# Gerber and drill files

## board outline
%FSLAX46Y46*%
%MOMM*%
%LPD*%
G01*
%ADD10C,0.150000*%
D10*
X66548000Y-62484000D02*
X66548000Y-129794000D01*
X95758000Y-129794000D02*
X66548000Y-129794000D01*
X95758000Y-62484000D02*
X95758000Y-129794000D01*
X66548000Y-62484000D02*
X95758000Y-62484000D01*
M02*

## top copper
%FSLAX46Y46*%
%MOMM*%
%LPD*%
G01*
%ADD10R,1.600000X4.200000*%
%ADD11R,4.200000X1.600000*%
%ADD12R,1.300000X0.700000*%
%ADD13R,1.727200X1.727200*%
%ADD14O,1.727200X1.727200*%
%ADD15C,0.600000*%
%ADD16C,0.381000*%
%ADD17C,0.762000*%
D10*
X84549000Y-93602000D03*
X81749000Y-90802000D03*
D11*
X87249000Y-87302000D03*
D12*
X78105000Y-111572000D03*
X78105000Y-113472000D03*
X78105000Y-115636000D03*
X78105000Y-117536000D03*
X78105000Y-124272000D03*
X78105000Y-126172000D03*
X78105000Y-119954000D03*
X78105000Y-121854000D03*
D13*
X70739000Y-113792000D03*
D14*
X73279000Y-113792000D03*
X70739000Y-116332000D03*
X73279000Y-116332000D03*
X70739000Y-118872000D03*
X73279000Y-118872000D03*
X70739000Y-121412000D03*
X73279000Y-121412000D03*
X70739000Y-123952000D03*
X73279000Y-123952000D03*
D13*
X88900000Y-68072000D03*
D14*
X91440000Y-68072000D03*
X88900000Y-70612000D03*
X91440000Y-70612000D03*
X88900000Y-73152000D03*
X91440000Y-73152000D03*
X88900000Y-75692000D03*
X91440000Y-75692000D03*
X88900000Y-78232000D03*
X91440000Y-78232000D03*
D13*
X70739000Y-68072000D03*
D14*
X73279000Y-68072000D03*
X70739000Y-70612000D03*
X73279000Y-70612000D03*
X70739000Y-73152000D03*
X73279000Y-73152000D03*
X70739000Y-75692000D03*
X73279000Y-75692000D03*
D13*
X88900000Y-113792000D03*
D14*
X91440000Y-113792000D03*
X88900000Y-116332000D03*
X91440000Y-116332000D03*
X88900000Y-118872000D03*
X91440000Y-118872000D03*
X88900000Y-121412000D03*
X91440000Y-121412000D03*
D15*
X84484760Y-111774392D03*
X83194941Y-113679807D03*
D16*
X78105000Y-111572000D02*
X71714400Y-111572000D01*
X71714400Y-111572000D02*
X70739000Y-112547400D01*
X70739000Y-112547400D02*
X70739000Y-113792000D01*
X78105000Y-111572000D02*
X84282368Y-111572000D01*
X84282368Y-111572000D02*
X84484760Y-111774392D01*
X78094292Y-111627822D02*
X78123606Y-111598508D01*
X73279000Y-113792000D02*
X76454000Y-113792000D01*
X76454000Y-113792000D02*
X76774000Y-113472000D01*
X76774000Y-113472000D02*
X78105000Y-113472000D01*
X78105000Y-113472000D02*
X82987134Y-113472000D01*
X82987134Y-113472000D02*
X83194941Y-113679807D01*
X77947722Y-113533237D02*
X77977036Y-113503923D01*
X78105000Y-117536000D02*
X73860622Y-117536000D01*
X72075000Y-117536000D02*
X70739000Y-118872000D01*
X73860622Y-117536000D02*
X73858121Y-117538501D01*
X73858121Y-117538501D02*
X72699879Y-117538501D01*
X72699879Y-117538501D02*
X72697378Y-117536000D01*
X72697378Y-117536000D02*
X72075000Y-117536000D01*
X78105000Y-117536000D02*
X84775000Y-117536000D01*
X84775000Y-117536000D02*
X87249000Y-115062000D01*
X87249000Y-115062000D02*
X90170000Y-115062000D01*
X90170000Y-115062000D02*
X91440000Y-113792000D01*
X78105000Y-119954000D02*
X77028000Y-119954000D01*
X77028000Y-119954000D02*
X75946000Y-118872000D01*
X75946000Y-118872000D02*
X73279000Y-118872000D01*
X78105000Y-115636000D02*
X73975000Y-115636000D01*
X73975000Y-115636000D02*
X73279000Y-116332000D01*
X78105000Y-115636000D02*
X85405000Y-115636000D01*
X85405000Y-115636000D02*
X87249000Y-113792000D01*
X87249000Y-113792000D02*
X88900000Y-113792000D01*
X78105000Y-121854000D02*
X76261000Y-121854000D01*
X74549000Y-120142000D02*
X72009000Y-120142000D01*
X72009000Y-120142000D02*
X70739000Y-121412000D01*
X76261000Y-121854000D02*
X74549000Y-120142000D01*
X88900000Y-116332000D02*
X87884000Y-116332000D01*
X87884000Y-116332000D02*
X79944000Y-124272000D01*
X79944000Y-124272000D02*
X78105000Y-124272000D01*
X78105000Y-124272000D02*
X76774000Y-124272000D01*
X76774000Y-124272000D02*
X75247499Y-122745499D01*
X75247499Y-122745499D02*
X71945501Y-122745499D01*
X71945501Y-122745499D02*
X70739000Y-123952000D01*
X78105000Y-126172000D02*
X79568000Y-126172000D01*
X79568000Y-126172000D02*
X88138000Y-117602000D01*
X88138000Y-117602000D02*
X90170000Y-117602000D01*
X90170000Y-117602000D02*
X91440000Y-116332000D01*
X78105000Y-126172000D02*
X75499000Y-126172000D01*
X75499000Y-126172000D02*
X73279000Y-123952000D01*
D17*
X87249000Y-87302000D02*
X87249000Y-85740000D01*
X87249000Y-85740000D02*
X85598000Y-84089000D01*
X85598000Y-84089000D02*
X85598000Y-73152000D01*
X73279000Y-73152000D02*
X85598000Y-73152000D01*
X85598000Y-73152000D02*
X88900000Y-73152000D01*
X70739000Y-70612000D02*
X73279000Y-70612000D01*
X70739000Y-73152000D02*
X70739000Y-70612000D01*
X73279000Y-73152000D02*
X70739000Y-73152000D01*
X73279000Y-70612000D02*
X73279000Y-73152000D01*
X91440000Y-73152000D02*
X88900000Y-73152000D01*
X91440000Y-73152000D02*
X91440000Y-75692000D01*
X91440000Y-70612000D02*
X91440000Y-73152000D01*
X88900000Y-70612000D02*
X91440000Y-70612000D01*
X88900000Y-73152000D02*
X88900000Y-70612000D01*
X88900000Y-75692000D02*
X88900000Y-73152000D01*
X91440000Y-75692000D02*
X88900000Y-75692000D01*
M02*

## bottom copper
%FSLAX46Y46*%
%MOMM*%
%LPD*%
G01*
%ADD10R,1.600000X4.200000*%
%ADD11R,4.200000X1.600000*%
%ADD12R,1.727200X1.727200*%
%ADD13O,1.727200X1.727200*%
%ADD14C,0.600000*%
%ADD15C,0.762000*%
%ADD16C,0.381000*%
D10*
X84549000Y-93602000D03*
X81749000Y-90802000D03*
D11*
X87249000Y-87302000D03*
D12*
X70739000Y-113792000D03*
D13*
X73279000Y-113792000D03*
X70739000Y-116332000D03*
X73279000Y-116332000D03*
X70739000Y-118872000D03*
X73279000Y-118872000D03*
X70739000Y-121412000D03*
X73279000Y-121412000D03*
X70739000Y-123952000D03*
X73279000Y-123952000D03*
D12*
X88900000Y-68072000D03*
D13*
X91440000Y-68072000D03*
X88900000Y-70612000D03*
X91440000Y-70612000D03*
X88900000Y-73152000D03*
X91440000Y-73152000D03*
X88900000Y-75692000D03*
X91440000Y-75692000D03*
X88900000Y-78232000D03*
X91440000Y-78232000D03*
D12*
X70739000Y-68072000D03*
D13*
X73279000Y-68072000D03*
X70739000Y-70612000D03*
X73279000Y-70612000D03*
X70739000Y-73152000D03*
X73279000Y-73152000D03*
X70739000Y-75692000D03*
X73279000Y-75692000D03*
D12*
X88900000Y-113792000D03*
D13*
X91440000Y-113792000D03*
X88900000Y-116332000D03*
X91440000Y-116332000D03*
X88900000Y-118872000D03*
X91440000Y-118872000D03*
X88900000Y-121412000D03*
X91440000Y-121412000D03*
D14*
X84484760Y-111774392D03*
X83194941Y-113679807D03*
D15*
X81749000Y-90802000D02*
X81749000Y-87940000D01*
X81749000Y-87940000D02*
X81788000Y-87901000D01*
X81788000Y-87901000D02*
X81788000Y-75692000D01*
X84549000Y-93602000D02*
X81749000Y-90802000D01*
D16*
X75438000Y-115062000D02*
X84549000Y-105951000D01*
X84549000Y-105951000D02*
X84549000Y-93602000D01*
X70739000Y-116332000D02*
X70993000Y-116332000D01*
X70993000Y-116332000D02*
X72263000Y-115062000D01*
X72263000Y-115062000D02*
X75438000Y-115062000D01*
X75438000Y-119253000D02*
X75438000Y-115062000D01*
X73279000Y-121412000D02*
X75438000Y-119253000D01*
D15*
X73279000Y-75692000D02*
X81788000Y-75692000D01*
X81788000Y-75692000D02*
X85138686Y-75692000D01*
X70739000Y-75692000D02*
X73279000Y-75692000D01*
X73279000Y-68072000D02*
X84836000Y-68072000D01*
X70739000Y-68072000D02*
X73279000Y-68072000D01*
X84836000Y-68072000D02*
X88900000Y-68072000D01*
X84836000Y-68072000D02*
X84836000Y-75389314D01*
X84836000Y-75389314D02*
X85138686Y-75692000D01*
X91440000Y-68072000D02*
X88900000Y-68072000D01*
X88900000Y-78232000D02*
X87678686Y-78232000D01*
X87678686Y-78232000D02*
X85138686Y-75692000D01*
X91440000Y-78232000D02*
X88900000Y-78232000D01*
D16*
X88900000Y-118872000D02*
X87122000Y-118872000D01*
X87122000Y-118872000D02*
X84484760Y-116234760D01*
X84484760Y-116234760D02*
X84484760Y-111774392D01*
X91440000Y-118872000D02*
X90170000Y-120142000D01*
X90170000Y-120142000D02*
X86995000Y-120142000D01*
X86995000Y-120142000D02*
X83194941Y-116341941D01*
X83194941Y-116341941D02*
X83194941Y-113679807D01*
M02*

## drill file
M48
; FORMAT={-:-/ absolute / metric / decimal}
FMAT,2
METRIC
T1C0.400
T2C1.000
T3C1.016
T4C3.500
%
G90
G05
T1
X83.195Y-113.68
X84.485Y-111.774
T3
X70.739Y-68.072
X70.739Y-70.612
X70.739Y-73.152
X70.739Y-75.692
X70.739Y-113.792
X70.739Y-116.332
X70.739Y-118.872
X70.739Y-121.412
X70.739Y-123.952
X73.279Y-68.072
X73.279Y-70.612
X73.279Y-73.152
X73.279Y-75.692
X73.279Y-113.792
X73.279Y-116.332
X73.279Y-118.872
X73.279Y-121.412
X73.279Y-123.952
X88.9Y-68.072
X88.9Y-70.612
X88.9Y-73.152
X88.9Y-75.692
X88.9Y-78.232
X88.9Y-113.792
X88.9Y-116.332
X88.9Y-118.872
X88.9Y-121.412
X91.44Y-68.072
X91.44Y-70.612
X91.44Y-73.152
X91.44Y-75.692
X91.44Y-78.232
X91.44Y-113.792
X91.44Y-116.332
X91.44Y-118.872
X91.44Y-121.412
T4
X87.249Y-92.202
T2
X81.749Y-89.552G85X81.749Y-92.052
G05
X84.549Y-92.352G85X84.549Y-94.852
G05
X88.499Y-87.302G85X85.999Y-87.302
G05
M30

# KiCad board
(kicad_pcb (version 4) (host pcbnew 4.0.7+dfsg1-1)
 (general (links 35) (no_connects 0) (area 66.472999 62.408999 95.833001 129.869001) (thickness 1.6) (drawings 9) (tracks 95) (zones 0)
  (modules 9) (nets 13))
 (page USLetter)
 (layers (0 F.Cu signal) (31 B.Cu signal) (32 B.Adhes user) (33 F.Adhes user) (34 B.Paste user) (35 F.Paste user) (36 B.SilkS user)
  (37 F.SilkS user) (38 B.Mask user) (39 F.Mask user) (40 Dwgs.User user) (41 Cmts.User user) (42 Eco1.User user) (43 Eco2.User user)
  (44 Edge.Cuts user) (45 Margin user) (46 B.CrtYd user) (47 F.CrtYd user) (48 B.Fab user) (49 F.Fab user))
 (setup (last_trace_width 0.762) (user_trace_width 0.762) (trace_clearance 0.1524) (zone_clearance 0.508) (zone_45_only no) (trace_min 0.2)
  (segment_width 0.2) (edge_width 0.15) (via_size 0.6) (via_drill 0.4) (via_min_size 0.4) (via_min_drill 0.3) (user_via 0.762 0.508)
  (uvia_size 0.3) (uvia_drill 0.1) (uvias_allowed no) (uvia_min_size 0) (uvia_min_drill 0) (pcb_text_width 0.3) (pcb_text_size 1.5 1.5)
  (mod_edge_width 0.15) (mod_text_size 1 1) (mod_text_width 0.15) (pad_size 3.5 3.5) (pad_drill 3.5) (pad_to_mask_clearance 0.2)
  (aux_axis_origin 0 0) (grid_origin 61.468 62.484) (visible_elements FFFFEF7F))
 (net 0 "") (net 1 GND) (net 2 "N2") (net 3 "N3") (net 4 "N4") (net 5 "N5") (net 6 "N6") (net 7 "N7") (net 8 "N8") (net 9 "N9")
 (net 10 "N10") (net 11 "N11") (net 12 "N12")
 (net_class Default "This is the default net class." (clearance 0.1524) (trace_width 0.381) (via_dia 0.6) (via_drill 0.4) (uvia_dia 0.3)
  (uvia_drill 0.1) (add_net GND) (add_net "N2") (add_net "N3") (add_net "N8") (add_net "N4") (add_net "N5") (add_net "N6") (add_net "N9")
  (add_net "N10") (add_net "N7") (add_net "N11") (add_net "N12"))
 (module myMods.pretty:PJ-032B (layer F.Cu) (at 87.249 87.302 270)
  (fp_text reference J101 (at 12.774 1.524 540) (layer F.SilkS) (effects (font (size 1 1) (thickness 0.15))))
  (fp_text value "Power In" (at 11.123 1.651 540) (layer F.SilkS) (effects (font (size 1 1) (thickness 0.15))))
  (pad 3 thru_hole rect (at 6.3 2.7) (size 1.6 4.2) (drill oval 1 3.5) (layers *.Cu *.Mask F.SilkS) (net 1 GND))
  (pad 2 thru_hole rect (at 3.5 5.5) (size 1.6 4.2) (drill oval 1 3.5) (layers *.Cu *.Mask F.SilkS) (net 1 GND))
  (pad 1 thru_hole rect (at 0 0 270) (size 1.6 4.2) (drill oval 1 3.5) (layers *.Cu *.Mask F.SilkS) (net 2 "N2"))
  (pad "" np_thru_hole circle (at 4.9 0) (size 3.5 3.5) (drill 3.5) (layers *.Cu *.Mask F.SilkS)))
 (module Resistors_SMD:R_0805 (layer F.Cu) (at 78.105 112.522 270)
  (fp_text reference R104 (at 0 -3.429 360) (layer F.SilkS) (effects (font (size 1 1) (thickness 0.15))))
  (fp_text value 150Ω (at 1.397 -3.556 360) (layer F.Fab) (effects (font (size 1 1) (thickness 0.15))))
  (pad 1 smd rect (at -0.95 0 270) (size 0.7 1.3) (layers F.Cu F.Paste F.Mask) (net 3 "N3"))
  (pad 2 smd rect (at 0.95 0 270) (size 0.7 1.3) (layers F.Cu F.Paste F.Mask) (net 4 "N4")))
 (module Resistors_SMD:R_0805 (layer F.Cu) (at 78.105 116.586 270)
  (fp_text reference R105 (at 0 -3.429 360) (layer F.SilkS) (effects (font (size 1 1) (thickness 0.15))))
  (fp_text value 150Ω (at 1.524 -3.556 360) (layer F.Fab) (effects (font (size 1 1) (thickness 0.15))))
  (pad 1 smd rect (at -0.95 0 270) (size 0.7 1.3) (layers F.Cu F.Paste F.Mask) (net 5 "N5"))
  (pad 2 smd rect (at 0.95 0 270) (size 0.7 1.3) (layers F.Cu F.Paste F.Mask) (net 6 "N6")))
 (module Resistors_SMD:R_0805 (layer F.Cu) (at 78.105 125.222 270)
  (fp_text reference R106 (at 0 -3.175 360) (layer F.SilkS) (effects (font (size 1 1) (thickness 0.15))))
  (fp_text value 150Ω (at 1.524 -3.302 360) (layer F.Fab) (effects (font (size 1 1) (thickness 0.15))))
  (pad 1 smd rect (at -0.95 0 270) (size 0.7 1.3) (layers F.Cu F.Paste F.Mask) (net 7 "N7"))
  (pad 2 smd rect (at 0.95 0 270) (size 0.7 1.3) (layers F.Cu F.Paste F.Mask) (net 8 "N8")))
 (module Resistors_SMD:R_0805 (layer F.Cu) (at 78.105 120.904 270)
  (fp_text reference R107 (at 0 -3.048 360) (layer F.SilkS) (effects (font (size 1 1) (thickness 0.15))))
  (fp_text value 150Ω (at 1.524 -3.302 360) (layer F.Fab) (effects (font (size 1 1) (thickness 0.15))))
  (pad 1 smd rect (at -0.95 0 270) (size 0.7 1.3) (layers F.Cu F.Paste F.Mask) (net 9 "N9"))
  (pad 2 smd rect (at 0.95 0 270) (size 0.7 1.3) (layers F.Cu F.Paste F.Mask) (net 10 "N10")))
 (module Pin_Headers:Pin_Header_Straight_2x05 (layer F.Cu) (at 70.739 113.792)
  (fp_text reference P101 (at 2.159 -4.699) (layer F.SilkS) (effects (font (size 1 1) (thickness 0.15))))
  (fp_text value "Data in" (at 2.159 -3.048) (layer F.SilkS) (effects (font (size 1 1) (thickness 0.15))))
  (pad 1 thru_hole rect (at 0 0) (size 1.7272 1.7272) (drill 1.016) (layers *.Cu *.Mask F.SilkS) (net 3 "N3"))
  (pad 2 thru_hole oval (at 2.54 0) (size 1.7272 1.7272) (drill 1.016) (layers *.Cu *.Mask F.SilkS) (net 4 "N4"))
  (pad 3 thru_hole oval (at 0 2.54) (size 1.7272 1.7272) (drill 1.016) (layers *.Cu *.Mask F.SilkS) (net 1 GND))
  (pad 4 thru_hole oval (at 2.54 2.54) (size 1.7272 1.7272) (drill 1.016) (layers *.Cu *.Mask F.SilkS) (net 5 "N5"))
  (pad 5 thru_hole oval (at 0 5.08) (size 1.7272 1.7272) (drill 1.016) (layers *.Cu *.Mask F.SilkS) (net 6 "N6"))
  (pad 6 thru_hole oval (at 2.54 5.08) (size 1.7272 1.7272) (drill 1.016) (layers *.Cu *.Mask F.SilkS) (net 9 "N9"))
  (pad 7 thru_hole oval (at 0 7.62) (size 1.7272 1.7272) (drill 1.016) (layers *.Cu *.Mask F.SilkS) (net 10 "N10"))
  (pad 8 thru_hole oval (at 2.54 7.62) (size 1.7272 1.7272) (drill 1.016) (layers *.Cu *.Mask F.SilkS) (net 1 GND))
  (pad 9 thru_hole oval (at 0 10.16) (size 1.7272 1.7272) (drill 1.016) (layers *.Cu *.Mask F.SilkS) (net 7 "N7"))
  (pad 10 thru_hole oval (at 2.54 10.16) (size 1.7272 1.7272) (drill 1.016) (layers *.Cu *.Mask F.SilkS) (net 8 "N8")))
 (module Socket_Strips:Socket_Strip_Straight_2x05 (layer B.Cu) (at 88.9 68.072 270)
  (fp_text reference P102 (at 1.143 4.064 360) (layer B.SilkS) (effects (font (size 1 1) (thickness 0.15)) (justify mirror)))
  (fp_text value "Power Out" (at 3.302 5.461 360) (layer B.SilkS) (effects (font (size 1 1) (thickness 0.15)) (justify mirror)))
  (pad 1 thru_hole rect (at 0 0 270) (size 1.7272 1.7272) (drill 1.016) (layers *.Cu *.Mask B.SilkS) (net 1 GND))
  (pad 2 thru_hole oval (at 0 -2.54 270) (size 1.7272 1.7272) (drill 1.016) (layers *.Cu *.Mask B.SilkS) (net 1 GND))
  (pad 3 thru_hole oval (at 2.54 0 270) (size 1.7272 1.7272) (drill 1.016) (layers *.Cu *.Mask B.SilkS) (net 2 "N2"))
  (pad 4 thru_hole oval (at 2.54 -2.54 270) (size 1.7272 1.7272) (drill 1.016) (layers *.Cu *.Mask B.SilkS) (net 2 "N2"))
  (pad 5 thru_hole oval (at 5.08 0 270) (size 1.7272 1.7272) (drill 1.016) (layers *.Cu *.Mask B.SilkS) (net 2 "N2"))
  (pad 6 thru_hole oval (at 5.08 -2.54 270) (size 1.7272 1.7272) (drill 1.016) (layers *.Cu *.Mask B.SilkS) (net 2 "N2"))
  (pad 7 thru_hole oval (at 7.62 0 270) (size 1.7272 1.7272) (drill 1.016) (layers *.Cu *.Mask B.SilkS) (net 2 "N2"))
  (pad 8 thru_hole oval (at 7.62 -2.54 270) (size 1.7272 1.7272) (drill 1.016) (layers *.Cu *.Mask B.SilkS) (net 2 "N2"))
  (pad 9 thru_hole oval (at 10.16 0 270) (size 1.7272 1.7272) (drill 1.016) (layers *.Cu *.Mask B.SilkS) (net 1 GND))
  (pad 10 thru_hole oval (at 10.16 -2.54 270) (size 1.7272 1.7272) (drill 1.016) (layers *.Cu *.Mask B.SilkS) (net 1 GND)))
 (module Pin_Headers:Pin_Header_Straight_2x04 (layer F.Cu) (at 70.739 68.072)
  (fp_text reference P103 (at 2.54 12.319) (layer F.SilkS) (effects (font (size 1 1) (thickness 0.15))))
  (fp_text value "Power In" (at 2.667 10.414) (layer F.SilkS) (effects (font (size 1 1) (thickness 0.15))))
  (pad 1 thru_hole rect (at 0 0) (size 1.7272 1.7272) (drill 1.016) (layers *.Cu *.Mask F.SilkS) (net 1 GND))
  (pad 2 thru_hole oval (at 2.54 0) (size 1.7272 1.7272) (drill 1.016) (layers *.Cu *.Mask F.SilkS) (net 1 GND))
  (pad 3 thru_hole oval (at 0 2.54) (size 1.7272 1.7272) (drill 1.016) (layers *.Cu *.Mask F.SilkS) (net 2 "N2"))
  (pad 4 thru_hole oval (at 2.54 2.54) (size 1.7272 1.7272) (drill 1.016) (layers *.Cu *.Mask F.SilkS) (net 2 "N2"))
  (pad 5 thru_hole oval (at 0 5.08) (size 1.7272 1.7272) (drill 1.016) (layers *.Cu *.Mask F.SilkS) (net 2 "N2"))
  (pad 6 thru_hole oval (at 2.54 5.08) (size 1.7272 1.7272) (drill 1.016) (layers *.Cu *.Mask F.SilkS) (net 2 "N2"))
  (pad 7 thru_hole oval (at 0 7.62) (size 1.7272 1.7272) (drill 1.016) (layers *.Cu *.Mask F.SilkS) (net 1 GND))
  (pad 8 thru_hole oval (at 2.54 7.62) (size 1.7272 1.7272) (drill 1.016) (layers *.Cu *.Mask F.SilkS) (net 1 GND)))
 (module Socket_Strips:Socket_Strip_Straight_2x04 (layer B.Cu) (at 88.9 113.792 270)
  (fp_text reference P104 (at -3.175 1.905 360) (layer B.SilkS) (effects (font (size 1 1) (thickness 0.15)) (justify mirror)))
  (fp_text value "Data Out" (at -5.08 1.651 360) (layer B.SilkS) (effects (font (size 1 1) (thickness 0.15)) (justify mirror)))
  (pad 1 thru_hole rect (at 0 0 270) (size 1.7272 1.7272) (drill 1.016) (layers *.Cu *.Mask B.SilkS) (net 5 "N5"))
  (pad 2 thru_hole oval (at 0 -2.54 270) (size 1.7272 1.7272) (drill 1.016) (layers *.Cu *.Mask B.SilkS) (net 6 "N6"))
  (pad 3 thru_hole oval (at 2.54 0 270) (size 1.7272 1.7272) (drill 1.016) (layers *.Cu *.Mask B.SilkS) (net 7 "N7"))
  (pad 4 thru_hole oval (at 2.54 -2.54 270) (size 1.7272 1.7272) (drill 1.016) (layers *.Cu *.Mask B.SilkS) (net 8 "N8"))
  (pad 5 thru_hole oval (at 5.08 0 270) (size 1.7272 1.7272) (drill 1.016) (layers *.Cu *.Mask B.SilkS) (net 3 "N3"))
  (pad 6 thru_hole oval (at 5.08 -2.54 270) (size 1.7272 1.7272) (drill 1.016) (layers *.Cu *.Mask B.SilkS) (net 4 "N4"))
  (pad 7 thru_hole oval (at 7.62 0 270) (size 1.7272 1.7272) (drill 1.016) (layers *.Cu *.Mask B.SilkS) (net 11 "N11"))
  (pad 8 thru_hole oval (at 7.62 -2.54 270) (size 1.7272 1.7272) (drill 1.016) (layers *.Cu *.Mask B.SilkS) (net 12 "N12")))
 (gr_line (start 66.548 62.484) (end 66.548 129.794) (angle 90) (layer Edge.Cuts) (width 0.15))
 (gr_line (start 95.758 129.794) (end 66.548 129.794) (angle 90) (layer Edge.Cuts) (width 0.15))
 (gr_line (start 95.758 62.484) (end 95.758 129.794) (angle 90) (layer Edge.Cuts) (width 0.15))
 (gr_line (start 66.548 62.484) (end 95.758 62.484) (angle 90) (layer Edge.Cuts) (width 0.15))
 (segment (start 81.749 90.802) (end 81.749 87.94) (width 0.762) (layer B.Cu) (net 1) (status 10))
 (segment (start 81.749 87.94) (end 81.788 87.901) (width 0.762) (layer B.Cu) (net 1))
 (segment (start 81.788 87.901) (end 81.788 75.692) (width 0.762) (layer B.Cu) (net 1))
 (segment (start 84.549 93.602) (end 81.749 90.802) (width 0.762) (layer B.Cu) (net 1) (status 30))
 (segment (start 75.438 115.062) (end 84.549 105.951) (width 0.381) (layer B.Cu) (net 1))
 (segment (start 84.549 105.951) (end 84.549 93.602) (width 0.381) (layer B.Cu) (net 1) (status 20))
 (segment (start 70.739 116.332) (end 70.993 116.332) (width 0.381) (layer B.Cu) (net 1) (status 30))
 (segment (start 70.993 116.332) (end 72.263 115.062) (width 0.381) (layer B.Cu) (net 1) (status 10))
 (segment (start 72.263 115.062) (end 75.438 115.062) (width 0.381) (layer B.Cu) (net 1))
 (segment (start 75.438 119.253) (end 75.438 115.062) (width 0.381) (layer B.Cu) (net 1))
 (segment (start 73.279 121.412) (end 75.438 119.253) (width 0.381) (layer B.Cu) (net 1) (status 10))
 (segment (start 73.279 75.692) (end 81.788 75.692) (width 0.762) (layer B.Cu) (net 1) (status 10))
 (segment (start 81.788 75.692) (end 85.138686 75.692) (width 0.762) (layer B.Cu) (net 1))
 (segment (start 70.739 75.692) (end 73.279 75.692) (width 0.762) (layer B.Cu) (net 1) (status 30))
 (segment (start 73.279 68.072) (end 84.836 68.072) (width 0.762) (layer B.Cu) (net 1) (status 10))
 (segment (start 70.739 68.072) (end 73.279 68.072) (width 0.762) (layer B.Cu) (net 1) (status 30))
 (segment (start 84.836 68.072) (end 88.9 68.072) (width 0.762) (layer B.Cu) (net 1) (status 20))
 (segment (start 84.836 68.072) (end 84.836 75.389314) (width 0.762) (layer B.Cu) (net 1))
 (segment (start 84.836 75.389314) (end 85.138686 75.692) (width 0.762) (layer B.Cu) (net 1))
 (segment (start 91.44 68.072) (end 88.9 68.072) (width 0.762) (layer B.Cu) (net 1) (status 30))
 (segment (start 88.9 78.232) (end 87.678686 78.232) (width 0.762) (layer B.Cu) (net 1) (status 10))
 (segment (start 87.678686 78.232) (end 85.138686 75.692) (width 0.762) (layer B.Cu) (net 1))
 (segment (start 91.44 78.232) (end 88.9 78.232) (width 0.762) (layer B.Cu) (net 1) (status 30))
 (segment (start 88.9 118.872) (end 87.122 118.872) (width 0.381) (layer B.Cu) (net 3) (status 10))
 (segment (start 87.122 118.872) (end 84.48476 116.23476) (width 0.381) (layer B.Cu) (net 3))
 (segment (start 84.48476 116.23476) (end 84.48476 111.774392) (width 0.381) (layer B.Cu) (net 3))
 (segment (start 78.105 111.572) (end 71.7144 111.572) (width 0.381) (layer F.Cu) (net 3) (status 10))
 (segment (start 71.7144 111.572) (end 70.739 112.5474) (width 0.381) (layer F.Cu) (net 3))
 (segment (start 70.739 112.5474) (end 70.739 113.792) (width 0.381) (layer F.Cu) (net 3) (status 20))
 (segment (start 78.105 111.572) (end 84.282368 111.572) (width 0.381) (layer F.Cu) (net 3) (status 10))
 (segment (start 84.282368 111.572) (end 84.48476 111.774392) (width 0.381) (layer F.Cu) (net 3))
 (segment (start 78.094292 111.627822) (end 78.123606 111.598508) (width 0.381) (layer F.Cu) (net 3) (status 30))
 (via (at 84.48476 111.774392) (size 0.6) (drill 0.4) (layers F.Cu B.Cu) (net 3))
 (segment (start 91.44 118.872) (end 90.17 120.142) (width 0.381) (layer B.Cu) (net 4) (status 10))
 (segment (start 90.17 120.142) (end 86.995 120.142) (width 0.381) (layer B.Cu) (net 4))
 (segment (start 86.995 120.142) (end 83.194941 116.341941) (width 0.381) (layer B.Cu) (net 4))
 (segment (start 83.194941 116.341941) (end 83.194941 113.679807) (width 0.381) (layer B.Cu) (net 4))
 (segment (start 73.279 113.792) (end 76.454 113.792) (width 0.381) (layer F.Cu) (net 4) (status 10))
 (segment (start 76.454 113.792) (end 76.774 113.472) (width 0.381) (layer F.Cu) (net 4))
 (segment (start 76.774 113.472) (end 78.105 113.472) (width 0.381) (layer F.Cu) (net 4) (status 20))
 (segment (start 78.105 113.472) (end 82.987134 113.472) (width 0.381) (layer F.Cu) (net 4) (status 10))
 (segment (start 82.987134 113.472) (end 83.194941 113.679807) (width 0.381) (layer F.Cu) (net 4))
 (segment (start 77.947722 113.533237) (end 77.977036 113.503923) (width 0.381) (layer F.Cu) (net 4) (status 30))
 (via (at 83.194941 113.679807) (size 0.6) (drill 0.4) (layers F.Cu B.Cu) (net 4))
 (segment (start 78.105 117.536) (end 73.860622 117.536) (width 0.381) (layer F.Cu) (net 6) (status 10))
 (segment (start 72.075 117.536) (end 70.739 118.872) (width 0.381) (layer F.Cu) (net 6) (status 20))
 (segment (start 73.860622 117.536) (end 73.858121 117.538501) (width 0.381) (layer F.Cu) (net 6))
 (segment (start 73.858121 117.538501) (end 72.699879 117.538501) (width 0.381) (layer F.Cu) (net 6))
 (segment (start 72.699879 117.538501) (end 72.697378 117.536) (width 0.381) (layer F.Cu) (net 6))
 (segment (start 72.697378 117.536) (end 72.075 117.536) (width 0.381) (layer F.Cu) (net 6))
 (segment (start 78.105 117.536) (end 84.775 117.536) (width 0.381) (layer F.Cu) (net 6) (status 10))
 (segment (start 84.775 117.536) (end 87.249 115.062) (width 0.381) (layer F.Cu) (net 6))
 (segment (start 87.249 115.062) (end 90.17 115.062) (width 0.381) (layer F.Cu) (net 6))
 (segment (start 90.17 115.062) (end 91.44 113.792) (width 0.381) (layer F.Cu) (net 6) (status 20))
 (segment (start 78.105 119.954) (end 77.028 119.954) (width 0.381) (layer F.Cu) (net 9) (status 10))
 (segment (start 77.028 119.954) (end 75.946 118.872) (width 0.381) (layer F.Cu) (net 9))
 (segment (start 75.946 118.872) (end 73.279 118.872) (width 0.381) (layer F.Cu) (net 9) (status 20))
 (segment (start 78.105 115.636) (end 73.975 115.636) (width 0.381) (layer F.Cu) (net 5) (status 10))
 (segment (start 73.975 115.636) (end 73.279 116.332) (width 0.381) (layer F.Cu) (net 5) (status 20))
 (segment (start 78.105 115.636) (end 85.405 115.636) (width 0.381) (layer F.Cu) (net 5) (status 10))
 (segment (start 85.405 115.636) (end 87.249 113.792) (width 0.381) (layer F.Cu) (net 5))
 (segment (start 87.249 113.792) (end 88.9 113.792) (width 0.381) (layer F.Cu) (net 5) (status 20))
 (segment (start 78.105 121.854) (end 76.261 121.854) (width 0.381) (layer F.Cu) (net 10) (status 10))
 (segment (start 74.549 120.142) (end 72.009 120.142) (width 0.381) (layer F.Cu) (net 10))
 (segment (start 72.009 120.142) (end 70.739 121.412) (width 0.381) (layer F.Cu) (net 10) (status 20))
 (segment (start 76.261 121.854) (end 74.549 120.142) (width 0.381) (layer F.Cu) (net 10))
 (segment (start 88.9 116.332) (end 87.884 116.332) (width 0.381) (layer F.Cu) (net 7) (status 10))
 (segment (start 87.884 116.332) (end 79.944 124.272) (width 0.381) (layer F.Cu) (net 7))
 (segment (start 79.944 124.272) (end 78.105 124.272) (width 0.381) (layer F.Cu) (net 7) (status 20))
 (segment (start 78.105 124.272) (end 76.774 124.272) (width 0.381) (layer F.Cu) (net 7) (status 10))
 (segment (start 76.774 124.272) (end 75.247499 122.745499) (width 0.381) (layer F.Cu) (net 7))
 (segment (start 75.247499 122.745499) (end 71.945501 122.745499) (width 0.381) (layer F.Cu) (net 7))
 (segment (start 71.945501 122.745499) (end 70.739 123.952) (width 0.381) (layer F.Cu) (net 7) (status 20))
 (segment (start 78.105 126.172) (end 79.568 126.172) (width 0.381) (layer F.Cu) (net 8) (status 10))
 (segment (start 79.568 126.172) (end 88.138 117.602) (width 0.381) (layer F.Cu) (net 8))
 (segment (start 88.138 117.602) (end 90.17 117.602) (width 0.381) (layer F.Cu) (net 8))
 (segment (start 90.17 117.602) (end 91.44 116.332) (width 0.381) (layer F.Cu) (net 8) (status 20))
 (segment (start 78.105 126.172) (end 75.499 126.172) (width 0.381) (layer F.Cu) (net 8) (status 10))
 (segment (start 75.499 126.172) (end 73.279 123.952) (width 0.381) (layer F.Cu) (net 8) (status 20))
 (segment (start 87.249 87.302) (end 87.249 85.74) (width 0.762) (layer F.Cu) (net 2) (status 10))
 (segment (start 87.249 85.74) (end 85.598 84.089) (width 0.762) (layer F.Cu) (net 2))
 (segment (start 85.598 84.089) (end 85.598 73.152) (width 0.762) (layer F.Cu) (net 2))
 (segment (start 73.279 73.152) (end 85.598 73.152) (width 0.762) (layer F.Cu) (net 2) (status 10))
 (segment (start 85.598 73.152) (end 88.9 73.152) (width 0.762) (layer F.Cu) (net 2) (status 20))
 (segment (start 70.739 70.612) (end 73.279 70.612) (width 0.762) (layer F.Cu) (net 2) (status 30))
 (segment (start 70.739 73.152) (end 70.739 70.612) (width 0.762) (layer F.Cu) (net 2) (status 30))
 (segment (start 73.279 73.152) (end 70.739 73.152) (width 0.762) (layer F.Cu) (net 2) (status 30))
 (segment (start 73.279 70.612) (end 73.279 73.152) (width 0.762) (layer F.Cu) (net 2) (status 30))
 (segment (start 91.44 73.152) (end 88.9 73.152) (width 0.762) (layer F.Cu) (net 2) (status 30))
 (segment (start 91.44 73.152) (end 91.44 75.692) (width 0.762) (layer F.Cu) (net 2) (status 30))
 (segment (start 91.44 70.612) (end 91.44 73.152) (width 0.762) (layer F.Cu) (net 2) (status 30))
 (segment (start 88.9 70.612) (end 91.44 70.612) (width 0.762) (layer F.Cu) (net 2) (status 30))
 (segment (start 88.9 73.152) (end 88.9 70.612) (width 0.762) (layer F.Cu) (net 2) (status 30))
 (segment (start 88.9 75.692) (end 88.9 73.152) (width 0.762) (layer F.Cu) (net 2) (status 30))
 (segment (start 91.44 75.692) (end 88.9 75.692) (width 0.762) (layer F.Cu) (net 2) (status 30)))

